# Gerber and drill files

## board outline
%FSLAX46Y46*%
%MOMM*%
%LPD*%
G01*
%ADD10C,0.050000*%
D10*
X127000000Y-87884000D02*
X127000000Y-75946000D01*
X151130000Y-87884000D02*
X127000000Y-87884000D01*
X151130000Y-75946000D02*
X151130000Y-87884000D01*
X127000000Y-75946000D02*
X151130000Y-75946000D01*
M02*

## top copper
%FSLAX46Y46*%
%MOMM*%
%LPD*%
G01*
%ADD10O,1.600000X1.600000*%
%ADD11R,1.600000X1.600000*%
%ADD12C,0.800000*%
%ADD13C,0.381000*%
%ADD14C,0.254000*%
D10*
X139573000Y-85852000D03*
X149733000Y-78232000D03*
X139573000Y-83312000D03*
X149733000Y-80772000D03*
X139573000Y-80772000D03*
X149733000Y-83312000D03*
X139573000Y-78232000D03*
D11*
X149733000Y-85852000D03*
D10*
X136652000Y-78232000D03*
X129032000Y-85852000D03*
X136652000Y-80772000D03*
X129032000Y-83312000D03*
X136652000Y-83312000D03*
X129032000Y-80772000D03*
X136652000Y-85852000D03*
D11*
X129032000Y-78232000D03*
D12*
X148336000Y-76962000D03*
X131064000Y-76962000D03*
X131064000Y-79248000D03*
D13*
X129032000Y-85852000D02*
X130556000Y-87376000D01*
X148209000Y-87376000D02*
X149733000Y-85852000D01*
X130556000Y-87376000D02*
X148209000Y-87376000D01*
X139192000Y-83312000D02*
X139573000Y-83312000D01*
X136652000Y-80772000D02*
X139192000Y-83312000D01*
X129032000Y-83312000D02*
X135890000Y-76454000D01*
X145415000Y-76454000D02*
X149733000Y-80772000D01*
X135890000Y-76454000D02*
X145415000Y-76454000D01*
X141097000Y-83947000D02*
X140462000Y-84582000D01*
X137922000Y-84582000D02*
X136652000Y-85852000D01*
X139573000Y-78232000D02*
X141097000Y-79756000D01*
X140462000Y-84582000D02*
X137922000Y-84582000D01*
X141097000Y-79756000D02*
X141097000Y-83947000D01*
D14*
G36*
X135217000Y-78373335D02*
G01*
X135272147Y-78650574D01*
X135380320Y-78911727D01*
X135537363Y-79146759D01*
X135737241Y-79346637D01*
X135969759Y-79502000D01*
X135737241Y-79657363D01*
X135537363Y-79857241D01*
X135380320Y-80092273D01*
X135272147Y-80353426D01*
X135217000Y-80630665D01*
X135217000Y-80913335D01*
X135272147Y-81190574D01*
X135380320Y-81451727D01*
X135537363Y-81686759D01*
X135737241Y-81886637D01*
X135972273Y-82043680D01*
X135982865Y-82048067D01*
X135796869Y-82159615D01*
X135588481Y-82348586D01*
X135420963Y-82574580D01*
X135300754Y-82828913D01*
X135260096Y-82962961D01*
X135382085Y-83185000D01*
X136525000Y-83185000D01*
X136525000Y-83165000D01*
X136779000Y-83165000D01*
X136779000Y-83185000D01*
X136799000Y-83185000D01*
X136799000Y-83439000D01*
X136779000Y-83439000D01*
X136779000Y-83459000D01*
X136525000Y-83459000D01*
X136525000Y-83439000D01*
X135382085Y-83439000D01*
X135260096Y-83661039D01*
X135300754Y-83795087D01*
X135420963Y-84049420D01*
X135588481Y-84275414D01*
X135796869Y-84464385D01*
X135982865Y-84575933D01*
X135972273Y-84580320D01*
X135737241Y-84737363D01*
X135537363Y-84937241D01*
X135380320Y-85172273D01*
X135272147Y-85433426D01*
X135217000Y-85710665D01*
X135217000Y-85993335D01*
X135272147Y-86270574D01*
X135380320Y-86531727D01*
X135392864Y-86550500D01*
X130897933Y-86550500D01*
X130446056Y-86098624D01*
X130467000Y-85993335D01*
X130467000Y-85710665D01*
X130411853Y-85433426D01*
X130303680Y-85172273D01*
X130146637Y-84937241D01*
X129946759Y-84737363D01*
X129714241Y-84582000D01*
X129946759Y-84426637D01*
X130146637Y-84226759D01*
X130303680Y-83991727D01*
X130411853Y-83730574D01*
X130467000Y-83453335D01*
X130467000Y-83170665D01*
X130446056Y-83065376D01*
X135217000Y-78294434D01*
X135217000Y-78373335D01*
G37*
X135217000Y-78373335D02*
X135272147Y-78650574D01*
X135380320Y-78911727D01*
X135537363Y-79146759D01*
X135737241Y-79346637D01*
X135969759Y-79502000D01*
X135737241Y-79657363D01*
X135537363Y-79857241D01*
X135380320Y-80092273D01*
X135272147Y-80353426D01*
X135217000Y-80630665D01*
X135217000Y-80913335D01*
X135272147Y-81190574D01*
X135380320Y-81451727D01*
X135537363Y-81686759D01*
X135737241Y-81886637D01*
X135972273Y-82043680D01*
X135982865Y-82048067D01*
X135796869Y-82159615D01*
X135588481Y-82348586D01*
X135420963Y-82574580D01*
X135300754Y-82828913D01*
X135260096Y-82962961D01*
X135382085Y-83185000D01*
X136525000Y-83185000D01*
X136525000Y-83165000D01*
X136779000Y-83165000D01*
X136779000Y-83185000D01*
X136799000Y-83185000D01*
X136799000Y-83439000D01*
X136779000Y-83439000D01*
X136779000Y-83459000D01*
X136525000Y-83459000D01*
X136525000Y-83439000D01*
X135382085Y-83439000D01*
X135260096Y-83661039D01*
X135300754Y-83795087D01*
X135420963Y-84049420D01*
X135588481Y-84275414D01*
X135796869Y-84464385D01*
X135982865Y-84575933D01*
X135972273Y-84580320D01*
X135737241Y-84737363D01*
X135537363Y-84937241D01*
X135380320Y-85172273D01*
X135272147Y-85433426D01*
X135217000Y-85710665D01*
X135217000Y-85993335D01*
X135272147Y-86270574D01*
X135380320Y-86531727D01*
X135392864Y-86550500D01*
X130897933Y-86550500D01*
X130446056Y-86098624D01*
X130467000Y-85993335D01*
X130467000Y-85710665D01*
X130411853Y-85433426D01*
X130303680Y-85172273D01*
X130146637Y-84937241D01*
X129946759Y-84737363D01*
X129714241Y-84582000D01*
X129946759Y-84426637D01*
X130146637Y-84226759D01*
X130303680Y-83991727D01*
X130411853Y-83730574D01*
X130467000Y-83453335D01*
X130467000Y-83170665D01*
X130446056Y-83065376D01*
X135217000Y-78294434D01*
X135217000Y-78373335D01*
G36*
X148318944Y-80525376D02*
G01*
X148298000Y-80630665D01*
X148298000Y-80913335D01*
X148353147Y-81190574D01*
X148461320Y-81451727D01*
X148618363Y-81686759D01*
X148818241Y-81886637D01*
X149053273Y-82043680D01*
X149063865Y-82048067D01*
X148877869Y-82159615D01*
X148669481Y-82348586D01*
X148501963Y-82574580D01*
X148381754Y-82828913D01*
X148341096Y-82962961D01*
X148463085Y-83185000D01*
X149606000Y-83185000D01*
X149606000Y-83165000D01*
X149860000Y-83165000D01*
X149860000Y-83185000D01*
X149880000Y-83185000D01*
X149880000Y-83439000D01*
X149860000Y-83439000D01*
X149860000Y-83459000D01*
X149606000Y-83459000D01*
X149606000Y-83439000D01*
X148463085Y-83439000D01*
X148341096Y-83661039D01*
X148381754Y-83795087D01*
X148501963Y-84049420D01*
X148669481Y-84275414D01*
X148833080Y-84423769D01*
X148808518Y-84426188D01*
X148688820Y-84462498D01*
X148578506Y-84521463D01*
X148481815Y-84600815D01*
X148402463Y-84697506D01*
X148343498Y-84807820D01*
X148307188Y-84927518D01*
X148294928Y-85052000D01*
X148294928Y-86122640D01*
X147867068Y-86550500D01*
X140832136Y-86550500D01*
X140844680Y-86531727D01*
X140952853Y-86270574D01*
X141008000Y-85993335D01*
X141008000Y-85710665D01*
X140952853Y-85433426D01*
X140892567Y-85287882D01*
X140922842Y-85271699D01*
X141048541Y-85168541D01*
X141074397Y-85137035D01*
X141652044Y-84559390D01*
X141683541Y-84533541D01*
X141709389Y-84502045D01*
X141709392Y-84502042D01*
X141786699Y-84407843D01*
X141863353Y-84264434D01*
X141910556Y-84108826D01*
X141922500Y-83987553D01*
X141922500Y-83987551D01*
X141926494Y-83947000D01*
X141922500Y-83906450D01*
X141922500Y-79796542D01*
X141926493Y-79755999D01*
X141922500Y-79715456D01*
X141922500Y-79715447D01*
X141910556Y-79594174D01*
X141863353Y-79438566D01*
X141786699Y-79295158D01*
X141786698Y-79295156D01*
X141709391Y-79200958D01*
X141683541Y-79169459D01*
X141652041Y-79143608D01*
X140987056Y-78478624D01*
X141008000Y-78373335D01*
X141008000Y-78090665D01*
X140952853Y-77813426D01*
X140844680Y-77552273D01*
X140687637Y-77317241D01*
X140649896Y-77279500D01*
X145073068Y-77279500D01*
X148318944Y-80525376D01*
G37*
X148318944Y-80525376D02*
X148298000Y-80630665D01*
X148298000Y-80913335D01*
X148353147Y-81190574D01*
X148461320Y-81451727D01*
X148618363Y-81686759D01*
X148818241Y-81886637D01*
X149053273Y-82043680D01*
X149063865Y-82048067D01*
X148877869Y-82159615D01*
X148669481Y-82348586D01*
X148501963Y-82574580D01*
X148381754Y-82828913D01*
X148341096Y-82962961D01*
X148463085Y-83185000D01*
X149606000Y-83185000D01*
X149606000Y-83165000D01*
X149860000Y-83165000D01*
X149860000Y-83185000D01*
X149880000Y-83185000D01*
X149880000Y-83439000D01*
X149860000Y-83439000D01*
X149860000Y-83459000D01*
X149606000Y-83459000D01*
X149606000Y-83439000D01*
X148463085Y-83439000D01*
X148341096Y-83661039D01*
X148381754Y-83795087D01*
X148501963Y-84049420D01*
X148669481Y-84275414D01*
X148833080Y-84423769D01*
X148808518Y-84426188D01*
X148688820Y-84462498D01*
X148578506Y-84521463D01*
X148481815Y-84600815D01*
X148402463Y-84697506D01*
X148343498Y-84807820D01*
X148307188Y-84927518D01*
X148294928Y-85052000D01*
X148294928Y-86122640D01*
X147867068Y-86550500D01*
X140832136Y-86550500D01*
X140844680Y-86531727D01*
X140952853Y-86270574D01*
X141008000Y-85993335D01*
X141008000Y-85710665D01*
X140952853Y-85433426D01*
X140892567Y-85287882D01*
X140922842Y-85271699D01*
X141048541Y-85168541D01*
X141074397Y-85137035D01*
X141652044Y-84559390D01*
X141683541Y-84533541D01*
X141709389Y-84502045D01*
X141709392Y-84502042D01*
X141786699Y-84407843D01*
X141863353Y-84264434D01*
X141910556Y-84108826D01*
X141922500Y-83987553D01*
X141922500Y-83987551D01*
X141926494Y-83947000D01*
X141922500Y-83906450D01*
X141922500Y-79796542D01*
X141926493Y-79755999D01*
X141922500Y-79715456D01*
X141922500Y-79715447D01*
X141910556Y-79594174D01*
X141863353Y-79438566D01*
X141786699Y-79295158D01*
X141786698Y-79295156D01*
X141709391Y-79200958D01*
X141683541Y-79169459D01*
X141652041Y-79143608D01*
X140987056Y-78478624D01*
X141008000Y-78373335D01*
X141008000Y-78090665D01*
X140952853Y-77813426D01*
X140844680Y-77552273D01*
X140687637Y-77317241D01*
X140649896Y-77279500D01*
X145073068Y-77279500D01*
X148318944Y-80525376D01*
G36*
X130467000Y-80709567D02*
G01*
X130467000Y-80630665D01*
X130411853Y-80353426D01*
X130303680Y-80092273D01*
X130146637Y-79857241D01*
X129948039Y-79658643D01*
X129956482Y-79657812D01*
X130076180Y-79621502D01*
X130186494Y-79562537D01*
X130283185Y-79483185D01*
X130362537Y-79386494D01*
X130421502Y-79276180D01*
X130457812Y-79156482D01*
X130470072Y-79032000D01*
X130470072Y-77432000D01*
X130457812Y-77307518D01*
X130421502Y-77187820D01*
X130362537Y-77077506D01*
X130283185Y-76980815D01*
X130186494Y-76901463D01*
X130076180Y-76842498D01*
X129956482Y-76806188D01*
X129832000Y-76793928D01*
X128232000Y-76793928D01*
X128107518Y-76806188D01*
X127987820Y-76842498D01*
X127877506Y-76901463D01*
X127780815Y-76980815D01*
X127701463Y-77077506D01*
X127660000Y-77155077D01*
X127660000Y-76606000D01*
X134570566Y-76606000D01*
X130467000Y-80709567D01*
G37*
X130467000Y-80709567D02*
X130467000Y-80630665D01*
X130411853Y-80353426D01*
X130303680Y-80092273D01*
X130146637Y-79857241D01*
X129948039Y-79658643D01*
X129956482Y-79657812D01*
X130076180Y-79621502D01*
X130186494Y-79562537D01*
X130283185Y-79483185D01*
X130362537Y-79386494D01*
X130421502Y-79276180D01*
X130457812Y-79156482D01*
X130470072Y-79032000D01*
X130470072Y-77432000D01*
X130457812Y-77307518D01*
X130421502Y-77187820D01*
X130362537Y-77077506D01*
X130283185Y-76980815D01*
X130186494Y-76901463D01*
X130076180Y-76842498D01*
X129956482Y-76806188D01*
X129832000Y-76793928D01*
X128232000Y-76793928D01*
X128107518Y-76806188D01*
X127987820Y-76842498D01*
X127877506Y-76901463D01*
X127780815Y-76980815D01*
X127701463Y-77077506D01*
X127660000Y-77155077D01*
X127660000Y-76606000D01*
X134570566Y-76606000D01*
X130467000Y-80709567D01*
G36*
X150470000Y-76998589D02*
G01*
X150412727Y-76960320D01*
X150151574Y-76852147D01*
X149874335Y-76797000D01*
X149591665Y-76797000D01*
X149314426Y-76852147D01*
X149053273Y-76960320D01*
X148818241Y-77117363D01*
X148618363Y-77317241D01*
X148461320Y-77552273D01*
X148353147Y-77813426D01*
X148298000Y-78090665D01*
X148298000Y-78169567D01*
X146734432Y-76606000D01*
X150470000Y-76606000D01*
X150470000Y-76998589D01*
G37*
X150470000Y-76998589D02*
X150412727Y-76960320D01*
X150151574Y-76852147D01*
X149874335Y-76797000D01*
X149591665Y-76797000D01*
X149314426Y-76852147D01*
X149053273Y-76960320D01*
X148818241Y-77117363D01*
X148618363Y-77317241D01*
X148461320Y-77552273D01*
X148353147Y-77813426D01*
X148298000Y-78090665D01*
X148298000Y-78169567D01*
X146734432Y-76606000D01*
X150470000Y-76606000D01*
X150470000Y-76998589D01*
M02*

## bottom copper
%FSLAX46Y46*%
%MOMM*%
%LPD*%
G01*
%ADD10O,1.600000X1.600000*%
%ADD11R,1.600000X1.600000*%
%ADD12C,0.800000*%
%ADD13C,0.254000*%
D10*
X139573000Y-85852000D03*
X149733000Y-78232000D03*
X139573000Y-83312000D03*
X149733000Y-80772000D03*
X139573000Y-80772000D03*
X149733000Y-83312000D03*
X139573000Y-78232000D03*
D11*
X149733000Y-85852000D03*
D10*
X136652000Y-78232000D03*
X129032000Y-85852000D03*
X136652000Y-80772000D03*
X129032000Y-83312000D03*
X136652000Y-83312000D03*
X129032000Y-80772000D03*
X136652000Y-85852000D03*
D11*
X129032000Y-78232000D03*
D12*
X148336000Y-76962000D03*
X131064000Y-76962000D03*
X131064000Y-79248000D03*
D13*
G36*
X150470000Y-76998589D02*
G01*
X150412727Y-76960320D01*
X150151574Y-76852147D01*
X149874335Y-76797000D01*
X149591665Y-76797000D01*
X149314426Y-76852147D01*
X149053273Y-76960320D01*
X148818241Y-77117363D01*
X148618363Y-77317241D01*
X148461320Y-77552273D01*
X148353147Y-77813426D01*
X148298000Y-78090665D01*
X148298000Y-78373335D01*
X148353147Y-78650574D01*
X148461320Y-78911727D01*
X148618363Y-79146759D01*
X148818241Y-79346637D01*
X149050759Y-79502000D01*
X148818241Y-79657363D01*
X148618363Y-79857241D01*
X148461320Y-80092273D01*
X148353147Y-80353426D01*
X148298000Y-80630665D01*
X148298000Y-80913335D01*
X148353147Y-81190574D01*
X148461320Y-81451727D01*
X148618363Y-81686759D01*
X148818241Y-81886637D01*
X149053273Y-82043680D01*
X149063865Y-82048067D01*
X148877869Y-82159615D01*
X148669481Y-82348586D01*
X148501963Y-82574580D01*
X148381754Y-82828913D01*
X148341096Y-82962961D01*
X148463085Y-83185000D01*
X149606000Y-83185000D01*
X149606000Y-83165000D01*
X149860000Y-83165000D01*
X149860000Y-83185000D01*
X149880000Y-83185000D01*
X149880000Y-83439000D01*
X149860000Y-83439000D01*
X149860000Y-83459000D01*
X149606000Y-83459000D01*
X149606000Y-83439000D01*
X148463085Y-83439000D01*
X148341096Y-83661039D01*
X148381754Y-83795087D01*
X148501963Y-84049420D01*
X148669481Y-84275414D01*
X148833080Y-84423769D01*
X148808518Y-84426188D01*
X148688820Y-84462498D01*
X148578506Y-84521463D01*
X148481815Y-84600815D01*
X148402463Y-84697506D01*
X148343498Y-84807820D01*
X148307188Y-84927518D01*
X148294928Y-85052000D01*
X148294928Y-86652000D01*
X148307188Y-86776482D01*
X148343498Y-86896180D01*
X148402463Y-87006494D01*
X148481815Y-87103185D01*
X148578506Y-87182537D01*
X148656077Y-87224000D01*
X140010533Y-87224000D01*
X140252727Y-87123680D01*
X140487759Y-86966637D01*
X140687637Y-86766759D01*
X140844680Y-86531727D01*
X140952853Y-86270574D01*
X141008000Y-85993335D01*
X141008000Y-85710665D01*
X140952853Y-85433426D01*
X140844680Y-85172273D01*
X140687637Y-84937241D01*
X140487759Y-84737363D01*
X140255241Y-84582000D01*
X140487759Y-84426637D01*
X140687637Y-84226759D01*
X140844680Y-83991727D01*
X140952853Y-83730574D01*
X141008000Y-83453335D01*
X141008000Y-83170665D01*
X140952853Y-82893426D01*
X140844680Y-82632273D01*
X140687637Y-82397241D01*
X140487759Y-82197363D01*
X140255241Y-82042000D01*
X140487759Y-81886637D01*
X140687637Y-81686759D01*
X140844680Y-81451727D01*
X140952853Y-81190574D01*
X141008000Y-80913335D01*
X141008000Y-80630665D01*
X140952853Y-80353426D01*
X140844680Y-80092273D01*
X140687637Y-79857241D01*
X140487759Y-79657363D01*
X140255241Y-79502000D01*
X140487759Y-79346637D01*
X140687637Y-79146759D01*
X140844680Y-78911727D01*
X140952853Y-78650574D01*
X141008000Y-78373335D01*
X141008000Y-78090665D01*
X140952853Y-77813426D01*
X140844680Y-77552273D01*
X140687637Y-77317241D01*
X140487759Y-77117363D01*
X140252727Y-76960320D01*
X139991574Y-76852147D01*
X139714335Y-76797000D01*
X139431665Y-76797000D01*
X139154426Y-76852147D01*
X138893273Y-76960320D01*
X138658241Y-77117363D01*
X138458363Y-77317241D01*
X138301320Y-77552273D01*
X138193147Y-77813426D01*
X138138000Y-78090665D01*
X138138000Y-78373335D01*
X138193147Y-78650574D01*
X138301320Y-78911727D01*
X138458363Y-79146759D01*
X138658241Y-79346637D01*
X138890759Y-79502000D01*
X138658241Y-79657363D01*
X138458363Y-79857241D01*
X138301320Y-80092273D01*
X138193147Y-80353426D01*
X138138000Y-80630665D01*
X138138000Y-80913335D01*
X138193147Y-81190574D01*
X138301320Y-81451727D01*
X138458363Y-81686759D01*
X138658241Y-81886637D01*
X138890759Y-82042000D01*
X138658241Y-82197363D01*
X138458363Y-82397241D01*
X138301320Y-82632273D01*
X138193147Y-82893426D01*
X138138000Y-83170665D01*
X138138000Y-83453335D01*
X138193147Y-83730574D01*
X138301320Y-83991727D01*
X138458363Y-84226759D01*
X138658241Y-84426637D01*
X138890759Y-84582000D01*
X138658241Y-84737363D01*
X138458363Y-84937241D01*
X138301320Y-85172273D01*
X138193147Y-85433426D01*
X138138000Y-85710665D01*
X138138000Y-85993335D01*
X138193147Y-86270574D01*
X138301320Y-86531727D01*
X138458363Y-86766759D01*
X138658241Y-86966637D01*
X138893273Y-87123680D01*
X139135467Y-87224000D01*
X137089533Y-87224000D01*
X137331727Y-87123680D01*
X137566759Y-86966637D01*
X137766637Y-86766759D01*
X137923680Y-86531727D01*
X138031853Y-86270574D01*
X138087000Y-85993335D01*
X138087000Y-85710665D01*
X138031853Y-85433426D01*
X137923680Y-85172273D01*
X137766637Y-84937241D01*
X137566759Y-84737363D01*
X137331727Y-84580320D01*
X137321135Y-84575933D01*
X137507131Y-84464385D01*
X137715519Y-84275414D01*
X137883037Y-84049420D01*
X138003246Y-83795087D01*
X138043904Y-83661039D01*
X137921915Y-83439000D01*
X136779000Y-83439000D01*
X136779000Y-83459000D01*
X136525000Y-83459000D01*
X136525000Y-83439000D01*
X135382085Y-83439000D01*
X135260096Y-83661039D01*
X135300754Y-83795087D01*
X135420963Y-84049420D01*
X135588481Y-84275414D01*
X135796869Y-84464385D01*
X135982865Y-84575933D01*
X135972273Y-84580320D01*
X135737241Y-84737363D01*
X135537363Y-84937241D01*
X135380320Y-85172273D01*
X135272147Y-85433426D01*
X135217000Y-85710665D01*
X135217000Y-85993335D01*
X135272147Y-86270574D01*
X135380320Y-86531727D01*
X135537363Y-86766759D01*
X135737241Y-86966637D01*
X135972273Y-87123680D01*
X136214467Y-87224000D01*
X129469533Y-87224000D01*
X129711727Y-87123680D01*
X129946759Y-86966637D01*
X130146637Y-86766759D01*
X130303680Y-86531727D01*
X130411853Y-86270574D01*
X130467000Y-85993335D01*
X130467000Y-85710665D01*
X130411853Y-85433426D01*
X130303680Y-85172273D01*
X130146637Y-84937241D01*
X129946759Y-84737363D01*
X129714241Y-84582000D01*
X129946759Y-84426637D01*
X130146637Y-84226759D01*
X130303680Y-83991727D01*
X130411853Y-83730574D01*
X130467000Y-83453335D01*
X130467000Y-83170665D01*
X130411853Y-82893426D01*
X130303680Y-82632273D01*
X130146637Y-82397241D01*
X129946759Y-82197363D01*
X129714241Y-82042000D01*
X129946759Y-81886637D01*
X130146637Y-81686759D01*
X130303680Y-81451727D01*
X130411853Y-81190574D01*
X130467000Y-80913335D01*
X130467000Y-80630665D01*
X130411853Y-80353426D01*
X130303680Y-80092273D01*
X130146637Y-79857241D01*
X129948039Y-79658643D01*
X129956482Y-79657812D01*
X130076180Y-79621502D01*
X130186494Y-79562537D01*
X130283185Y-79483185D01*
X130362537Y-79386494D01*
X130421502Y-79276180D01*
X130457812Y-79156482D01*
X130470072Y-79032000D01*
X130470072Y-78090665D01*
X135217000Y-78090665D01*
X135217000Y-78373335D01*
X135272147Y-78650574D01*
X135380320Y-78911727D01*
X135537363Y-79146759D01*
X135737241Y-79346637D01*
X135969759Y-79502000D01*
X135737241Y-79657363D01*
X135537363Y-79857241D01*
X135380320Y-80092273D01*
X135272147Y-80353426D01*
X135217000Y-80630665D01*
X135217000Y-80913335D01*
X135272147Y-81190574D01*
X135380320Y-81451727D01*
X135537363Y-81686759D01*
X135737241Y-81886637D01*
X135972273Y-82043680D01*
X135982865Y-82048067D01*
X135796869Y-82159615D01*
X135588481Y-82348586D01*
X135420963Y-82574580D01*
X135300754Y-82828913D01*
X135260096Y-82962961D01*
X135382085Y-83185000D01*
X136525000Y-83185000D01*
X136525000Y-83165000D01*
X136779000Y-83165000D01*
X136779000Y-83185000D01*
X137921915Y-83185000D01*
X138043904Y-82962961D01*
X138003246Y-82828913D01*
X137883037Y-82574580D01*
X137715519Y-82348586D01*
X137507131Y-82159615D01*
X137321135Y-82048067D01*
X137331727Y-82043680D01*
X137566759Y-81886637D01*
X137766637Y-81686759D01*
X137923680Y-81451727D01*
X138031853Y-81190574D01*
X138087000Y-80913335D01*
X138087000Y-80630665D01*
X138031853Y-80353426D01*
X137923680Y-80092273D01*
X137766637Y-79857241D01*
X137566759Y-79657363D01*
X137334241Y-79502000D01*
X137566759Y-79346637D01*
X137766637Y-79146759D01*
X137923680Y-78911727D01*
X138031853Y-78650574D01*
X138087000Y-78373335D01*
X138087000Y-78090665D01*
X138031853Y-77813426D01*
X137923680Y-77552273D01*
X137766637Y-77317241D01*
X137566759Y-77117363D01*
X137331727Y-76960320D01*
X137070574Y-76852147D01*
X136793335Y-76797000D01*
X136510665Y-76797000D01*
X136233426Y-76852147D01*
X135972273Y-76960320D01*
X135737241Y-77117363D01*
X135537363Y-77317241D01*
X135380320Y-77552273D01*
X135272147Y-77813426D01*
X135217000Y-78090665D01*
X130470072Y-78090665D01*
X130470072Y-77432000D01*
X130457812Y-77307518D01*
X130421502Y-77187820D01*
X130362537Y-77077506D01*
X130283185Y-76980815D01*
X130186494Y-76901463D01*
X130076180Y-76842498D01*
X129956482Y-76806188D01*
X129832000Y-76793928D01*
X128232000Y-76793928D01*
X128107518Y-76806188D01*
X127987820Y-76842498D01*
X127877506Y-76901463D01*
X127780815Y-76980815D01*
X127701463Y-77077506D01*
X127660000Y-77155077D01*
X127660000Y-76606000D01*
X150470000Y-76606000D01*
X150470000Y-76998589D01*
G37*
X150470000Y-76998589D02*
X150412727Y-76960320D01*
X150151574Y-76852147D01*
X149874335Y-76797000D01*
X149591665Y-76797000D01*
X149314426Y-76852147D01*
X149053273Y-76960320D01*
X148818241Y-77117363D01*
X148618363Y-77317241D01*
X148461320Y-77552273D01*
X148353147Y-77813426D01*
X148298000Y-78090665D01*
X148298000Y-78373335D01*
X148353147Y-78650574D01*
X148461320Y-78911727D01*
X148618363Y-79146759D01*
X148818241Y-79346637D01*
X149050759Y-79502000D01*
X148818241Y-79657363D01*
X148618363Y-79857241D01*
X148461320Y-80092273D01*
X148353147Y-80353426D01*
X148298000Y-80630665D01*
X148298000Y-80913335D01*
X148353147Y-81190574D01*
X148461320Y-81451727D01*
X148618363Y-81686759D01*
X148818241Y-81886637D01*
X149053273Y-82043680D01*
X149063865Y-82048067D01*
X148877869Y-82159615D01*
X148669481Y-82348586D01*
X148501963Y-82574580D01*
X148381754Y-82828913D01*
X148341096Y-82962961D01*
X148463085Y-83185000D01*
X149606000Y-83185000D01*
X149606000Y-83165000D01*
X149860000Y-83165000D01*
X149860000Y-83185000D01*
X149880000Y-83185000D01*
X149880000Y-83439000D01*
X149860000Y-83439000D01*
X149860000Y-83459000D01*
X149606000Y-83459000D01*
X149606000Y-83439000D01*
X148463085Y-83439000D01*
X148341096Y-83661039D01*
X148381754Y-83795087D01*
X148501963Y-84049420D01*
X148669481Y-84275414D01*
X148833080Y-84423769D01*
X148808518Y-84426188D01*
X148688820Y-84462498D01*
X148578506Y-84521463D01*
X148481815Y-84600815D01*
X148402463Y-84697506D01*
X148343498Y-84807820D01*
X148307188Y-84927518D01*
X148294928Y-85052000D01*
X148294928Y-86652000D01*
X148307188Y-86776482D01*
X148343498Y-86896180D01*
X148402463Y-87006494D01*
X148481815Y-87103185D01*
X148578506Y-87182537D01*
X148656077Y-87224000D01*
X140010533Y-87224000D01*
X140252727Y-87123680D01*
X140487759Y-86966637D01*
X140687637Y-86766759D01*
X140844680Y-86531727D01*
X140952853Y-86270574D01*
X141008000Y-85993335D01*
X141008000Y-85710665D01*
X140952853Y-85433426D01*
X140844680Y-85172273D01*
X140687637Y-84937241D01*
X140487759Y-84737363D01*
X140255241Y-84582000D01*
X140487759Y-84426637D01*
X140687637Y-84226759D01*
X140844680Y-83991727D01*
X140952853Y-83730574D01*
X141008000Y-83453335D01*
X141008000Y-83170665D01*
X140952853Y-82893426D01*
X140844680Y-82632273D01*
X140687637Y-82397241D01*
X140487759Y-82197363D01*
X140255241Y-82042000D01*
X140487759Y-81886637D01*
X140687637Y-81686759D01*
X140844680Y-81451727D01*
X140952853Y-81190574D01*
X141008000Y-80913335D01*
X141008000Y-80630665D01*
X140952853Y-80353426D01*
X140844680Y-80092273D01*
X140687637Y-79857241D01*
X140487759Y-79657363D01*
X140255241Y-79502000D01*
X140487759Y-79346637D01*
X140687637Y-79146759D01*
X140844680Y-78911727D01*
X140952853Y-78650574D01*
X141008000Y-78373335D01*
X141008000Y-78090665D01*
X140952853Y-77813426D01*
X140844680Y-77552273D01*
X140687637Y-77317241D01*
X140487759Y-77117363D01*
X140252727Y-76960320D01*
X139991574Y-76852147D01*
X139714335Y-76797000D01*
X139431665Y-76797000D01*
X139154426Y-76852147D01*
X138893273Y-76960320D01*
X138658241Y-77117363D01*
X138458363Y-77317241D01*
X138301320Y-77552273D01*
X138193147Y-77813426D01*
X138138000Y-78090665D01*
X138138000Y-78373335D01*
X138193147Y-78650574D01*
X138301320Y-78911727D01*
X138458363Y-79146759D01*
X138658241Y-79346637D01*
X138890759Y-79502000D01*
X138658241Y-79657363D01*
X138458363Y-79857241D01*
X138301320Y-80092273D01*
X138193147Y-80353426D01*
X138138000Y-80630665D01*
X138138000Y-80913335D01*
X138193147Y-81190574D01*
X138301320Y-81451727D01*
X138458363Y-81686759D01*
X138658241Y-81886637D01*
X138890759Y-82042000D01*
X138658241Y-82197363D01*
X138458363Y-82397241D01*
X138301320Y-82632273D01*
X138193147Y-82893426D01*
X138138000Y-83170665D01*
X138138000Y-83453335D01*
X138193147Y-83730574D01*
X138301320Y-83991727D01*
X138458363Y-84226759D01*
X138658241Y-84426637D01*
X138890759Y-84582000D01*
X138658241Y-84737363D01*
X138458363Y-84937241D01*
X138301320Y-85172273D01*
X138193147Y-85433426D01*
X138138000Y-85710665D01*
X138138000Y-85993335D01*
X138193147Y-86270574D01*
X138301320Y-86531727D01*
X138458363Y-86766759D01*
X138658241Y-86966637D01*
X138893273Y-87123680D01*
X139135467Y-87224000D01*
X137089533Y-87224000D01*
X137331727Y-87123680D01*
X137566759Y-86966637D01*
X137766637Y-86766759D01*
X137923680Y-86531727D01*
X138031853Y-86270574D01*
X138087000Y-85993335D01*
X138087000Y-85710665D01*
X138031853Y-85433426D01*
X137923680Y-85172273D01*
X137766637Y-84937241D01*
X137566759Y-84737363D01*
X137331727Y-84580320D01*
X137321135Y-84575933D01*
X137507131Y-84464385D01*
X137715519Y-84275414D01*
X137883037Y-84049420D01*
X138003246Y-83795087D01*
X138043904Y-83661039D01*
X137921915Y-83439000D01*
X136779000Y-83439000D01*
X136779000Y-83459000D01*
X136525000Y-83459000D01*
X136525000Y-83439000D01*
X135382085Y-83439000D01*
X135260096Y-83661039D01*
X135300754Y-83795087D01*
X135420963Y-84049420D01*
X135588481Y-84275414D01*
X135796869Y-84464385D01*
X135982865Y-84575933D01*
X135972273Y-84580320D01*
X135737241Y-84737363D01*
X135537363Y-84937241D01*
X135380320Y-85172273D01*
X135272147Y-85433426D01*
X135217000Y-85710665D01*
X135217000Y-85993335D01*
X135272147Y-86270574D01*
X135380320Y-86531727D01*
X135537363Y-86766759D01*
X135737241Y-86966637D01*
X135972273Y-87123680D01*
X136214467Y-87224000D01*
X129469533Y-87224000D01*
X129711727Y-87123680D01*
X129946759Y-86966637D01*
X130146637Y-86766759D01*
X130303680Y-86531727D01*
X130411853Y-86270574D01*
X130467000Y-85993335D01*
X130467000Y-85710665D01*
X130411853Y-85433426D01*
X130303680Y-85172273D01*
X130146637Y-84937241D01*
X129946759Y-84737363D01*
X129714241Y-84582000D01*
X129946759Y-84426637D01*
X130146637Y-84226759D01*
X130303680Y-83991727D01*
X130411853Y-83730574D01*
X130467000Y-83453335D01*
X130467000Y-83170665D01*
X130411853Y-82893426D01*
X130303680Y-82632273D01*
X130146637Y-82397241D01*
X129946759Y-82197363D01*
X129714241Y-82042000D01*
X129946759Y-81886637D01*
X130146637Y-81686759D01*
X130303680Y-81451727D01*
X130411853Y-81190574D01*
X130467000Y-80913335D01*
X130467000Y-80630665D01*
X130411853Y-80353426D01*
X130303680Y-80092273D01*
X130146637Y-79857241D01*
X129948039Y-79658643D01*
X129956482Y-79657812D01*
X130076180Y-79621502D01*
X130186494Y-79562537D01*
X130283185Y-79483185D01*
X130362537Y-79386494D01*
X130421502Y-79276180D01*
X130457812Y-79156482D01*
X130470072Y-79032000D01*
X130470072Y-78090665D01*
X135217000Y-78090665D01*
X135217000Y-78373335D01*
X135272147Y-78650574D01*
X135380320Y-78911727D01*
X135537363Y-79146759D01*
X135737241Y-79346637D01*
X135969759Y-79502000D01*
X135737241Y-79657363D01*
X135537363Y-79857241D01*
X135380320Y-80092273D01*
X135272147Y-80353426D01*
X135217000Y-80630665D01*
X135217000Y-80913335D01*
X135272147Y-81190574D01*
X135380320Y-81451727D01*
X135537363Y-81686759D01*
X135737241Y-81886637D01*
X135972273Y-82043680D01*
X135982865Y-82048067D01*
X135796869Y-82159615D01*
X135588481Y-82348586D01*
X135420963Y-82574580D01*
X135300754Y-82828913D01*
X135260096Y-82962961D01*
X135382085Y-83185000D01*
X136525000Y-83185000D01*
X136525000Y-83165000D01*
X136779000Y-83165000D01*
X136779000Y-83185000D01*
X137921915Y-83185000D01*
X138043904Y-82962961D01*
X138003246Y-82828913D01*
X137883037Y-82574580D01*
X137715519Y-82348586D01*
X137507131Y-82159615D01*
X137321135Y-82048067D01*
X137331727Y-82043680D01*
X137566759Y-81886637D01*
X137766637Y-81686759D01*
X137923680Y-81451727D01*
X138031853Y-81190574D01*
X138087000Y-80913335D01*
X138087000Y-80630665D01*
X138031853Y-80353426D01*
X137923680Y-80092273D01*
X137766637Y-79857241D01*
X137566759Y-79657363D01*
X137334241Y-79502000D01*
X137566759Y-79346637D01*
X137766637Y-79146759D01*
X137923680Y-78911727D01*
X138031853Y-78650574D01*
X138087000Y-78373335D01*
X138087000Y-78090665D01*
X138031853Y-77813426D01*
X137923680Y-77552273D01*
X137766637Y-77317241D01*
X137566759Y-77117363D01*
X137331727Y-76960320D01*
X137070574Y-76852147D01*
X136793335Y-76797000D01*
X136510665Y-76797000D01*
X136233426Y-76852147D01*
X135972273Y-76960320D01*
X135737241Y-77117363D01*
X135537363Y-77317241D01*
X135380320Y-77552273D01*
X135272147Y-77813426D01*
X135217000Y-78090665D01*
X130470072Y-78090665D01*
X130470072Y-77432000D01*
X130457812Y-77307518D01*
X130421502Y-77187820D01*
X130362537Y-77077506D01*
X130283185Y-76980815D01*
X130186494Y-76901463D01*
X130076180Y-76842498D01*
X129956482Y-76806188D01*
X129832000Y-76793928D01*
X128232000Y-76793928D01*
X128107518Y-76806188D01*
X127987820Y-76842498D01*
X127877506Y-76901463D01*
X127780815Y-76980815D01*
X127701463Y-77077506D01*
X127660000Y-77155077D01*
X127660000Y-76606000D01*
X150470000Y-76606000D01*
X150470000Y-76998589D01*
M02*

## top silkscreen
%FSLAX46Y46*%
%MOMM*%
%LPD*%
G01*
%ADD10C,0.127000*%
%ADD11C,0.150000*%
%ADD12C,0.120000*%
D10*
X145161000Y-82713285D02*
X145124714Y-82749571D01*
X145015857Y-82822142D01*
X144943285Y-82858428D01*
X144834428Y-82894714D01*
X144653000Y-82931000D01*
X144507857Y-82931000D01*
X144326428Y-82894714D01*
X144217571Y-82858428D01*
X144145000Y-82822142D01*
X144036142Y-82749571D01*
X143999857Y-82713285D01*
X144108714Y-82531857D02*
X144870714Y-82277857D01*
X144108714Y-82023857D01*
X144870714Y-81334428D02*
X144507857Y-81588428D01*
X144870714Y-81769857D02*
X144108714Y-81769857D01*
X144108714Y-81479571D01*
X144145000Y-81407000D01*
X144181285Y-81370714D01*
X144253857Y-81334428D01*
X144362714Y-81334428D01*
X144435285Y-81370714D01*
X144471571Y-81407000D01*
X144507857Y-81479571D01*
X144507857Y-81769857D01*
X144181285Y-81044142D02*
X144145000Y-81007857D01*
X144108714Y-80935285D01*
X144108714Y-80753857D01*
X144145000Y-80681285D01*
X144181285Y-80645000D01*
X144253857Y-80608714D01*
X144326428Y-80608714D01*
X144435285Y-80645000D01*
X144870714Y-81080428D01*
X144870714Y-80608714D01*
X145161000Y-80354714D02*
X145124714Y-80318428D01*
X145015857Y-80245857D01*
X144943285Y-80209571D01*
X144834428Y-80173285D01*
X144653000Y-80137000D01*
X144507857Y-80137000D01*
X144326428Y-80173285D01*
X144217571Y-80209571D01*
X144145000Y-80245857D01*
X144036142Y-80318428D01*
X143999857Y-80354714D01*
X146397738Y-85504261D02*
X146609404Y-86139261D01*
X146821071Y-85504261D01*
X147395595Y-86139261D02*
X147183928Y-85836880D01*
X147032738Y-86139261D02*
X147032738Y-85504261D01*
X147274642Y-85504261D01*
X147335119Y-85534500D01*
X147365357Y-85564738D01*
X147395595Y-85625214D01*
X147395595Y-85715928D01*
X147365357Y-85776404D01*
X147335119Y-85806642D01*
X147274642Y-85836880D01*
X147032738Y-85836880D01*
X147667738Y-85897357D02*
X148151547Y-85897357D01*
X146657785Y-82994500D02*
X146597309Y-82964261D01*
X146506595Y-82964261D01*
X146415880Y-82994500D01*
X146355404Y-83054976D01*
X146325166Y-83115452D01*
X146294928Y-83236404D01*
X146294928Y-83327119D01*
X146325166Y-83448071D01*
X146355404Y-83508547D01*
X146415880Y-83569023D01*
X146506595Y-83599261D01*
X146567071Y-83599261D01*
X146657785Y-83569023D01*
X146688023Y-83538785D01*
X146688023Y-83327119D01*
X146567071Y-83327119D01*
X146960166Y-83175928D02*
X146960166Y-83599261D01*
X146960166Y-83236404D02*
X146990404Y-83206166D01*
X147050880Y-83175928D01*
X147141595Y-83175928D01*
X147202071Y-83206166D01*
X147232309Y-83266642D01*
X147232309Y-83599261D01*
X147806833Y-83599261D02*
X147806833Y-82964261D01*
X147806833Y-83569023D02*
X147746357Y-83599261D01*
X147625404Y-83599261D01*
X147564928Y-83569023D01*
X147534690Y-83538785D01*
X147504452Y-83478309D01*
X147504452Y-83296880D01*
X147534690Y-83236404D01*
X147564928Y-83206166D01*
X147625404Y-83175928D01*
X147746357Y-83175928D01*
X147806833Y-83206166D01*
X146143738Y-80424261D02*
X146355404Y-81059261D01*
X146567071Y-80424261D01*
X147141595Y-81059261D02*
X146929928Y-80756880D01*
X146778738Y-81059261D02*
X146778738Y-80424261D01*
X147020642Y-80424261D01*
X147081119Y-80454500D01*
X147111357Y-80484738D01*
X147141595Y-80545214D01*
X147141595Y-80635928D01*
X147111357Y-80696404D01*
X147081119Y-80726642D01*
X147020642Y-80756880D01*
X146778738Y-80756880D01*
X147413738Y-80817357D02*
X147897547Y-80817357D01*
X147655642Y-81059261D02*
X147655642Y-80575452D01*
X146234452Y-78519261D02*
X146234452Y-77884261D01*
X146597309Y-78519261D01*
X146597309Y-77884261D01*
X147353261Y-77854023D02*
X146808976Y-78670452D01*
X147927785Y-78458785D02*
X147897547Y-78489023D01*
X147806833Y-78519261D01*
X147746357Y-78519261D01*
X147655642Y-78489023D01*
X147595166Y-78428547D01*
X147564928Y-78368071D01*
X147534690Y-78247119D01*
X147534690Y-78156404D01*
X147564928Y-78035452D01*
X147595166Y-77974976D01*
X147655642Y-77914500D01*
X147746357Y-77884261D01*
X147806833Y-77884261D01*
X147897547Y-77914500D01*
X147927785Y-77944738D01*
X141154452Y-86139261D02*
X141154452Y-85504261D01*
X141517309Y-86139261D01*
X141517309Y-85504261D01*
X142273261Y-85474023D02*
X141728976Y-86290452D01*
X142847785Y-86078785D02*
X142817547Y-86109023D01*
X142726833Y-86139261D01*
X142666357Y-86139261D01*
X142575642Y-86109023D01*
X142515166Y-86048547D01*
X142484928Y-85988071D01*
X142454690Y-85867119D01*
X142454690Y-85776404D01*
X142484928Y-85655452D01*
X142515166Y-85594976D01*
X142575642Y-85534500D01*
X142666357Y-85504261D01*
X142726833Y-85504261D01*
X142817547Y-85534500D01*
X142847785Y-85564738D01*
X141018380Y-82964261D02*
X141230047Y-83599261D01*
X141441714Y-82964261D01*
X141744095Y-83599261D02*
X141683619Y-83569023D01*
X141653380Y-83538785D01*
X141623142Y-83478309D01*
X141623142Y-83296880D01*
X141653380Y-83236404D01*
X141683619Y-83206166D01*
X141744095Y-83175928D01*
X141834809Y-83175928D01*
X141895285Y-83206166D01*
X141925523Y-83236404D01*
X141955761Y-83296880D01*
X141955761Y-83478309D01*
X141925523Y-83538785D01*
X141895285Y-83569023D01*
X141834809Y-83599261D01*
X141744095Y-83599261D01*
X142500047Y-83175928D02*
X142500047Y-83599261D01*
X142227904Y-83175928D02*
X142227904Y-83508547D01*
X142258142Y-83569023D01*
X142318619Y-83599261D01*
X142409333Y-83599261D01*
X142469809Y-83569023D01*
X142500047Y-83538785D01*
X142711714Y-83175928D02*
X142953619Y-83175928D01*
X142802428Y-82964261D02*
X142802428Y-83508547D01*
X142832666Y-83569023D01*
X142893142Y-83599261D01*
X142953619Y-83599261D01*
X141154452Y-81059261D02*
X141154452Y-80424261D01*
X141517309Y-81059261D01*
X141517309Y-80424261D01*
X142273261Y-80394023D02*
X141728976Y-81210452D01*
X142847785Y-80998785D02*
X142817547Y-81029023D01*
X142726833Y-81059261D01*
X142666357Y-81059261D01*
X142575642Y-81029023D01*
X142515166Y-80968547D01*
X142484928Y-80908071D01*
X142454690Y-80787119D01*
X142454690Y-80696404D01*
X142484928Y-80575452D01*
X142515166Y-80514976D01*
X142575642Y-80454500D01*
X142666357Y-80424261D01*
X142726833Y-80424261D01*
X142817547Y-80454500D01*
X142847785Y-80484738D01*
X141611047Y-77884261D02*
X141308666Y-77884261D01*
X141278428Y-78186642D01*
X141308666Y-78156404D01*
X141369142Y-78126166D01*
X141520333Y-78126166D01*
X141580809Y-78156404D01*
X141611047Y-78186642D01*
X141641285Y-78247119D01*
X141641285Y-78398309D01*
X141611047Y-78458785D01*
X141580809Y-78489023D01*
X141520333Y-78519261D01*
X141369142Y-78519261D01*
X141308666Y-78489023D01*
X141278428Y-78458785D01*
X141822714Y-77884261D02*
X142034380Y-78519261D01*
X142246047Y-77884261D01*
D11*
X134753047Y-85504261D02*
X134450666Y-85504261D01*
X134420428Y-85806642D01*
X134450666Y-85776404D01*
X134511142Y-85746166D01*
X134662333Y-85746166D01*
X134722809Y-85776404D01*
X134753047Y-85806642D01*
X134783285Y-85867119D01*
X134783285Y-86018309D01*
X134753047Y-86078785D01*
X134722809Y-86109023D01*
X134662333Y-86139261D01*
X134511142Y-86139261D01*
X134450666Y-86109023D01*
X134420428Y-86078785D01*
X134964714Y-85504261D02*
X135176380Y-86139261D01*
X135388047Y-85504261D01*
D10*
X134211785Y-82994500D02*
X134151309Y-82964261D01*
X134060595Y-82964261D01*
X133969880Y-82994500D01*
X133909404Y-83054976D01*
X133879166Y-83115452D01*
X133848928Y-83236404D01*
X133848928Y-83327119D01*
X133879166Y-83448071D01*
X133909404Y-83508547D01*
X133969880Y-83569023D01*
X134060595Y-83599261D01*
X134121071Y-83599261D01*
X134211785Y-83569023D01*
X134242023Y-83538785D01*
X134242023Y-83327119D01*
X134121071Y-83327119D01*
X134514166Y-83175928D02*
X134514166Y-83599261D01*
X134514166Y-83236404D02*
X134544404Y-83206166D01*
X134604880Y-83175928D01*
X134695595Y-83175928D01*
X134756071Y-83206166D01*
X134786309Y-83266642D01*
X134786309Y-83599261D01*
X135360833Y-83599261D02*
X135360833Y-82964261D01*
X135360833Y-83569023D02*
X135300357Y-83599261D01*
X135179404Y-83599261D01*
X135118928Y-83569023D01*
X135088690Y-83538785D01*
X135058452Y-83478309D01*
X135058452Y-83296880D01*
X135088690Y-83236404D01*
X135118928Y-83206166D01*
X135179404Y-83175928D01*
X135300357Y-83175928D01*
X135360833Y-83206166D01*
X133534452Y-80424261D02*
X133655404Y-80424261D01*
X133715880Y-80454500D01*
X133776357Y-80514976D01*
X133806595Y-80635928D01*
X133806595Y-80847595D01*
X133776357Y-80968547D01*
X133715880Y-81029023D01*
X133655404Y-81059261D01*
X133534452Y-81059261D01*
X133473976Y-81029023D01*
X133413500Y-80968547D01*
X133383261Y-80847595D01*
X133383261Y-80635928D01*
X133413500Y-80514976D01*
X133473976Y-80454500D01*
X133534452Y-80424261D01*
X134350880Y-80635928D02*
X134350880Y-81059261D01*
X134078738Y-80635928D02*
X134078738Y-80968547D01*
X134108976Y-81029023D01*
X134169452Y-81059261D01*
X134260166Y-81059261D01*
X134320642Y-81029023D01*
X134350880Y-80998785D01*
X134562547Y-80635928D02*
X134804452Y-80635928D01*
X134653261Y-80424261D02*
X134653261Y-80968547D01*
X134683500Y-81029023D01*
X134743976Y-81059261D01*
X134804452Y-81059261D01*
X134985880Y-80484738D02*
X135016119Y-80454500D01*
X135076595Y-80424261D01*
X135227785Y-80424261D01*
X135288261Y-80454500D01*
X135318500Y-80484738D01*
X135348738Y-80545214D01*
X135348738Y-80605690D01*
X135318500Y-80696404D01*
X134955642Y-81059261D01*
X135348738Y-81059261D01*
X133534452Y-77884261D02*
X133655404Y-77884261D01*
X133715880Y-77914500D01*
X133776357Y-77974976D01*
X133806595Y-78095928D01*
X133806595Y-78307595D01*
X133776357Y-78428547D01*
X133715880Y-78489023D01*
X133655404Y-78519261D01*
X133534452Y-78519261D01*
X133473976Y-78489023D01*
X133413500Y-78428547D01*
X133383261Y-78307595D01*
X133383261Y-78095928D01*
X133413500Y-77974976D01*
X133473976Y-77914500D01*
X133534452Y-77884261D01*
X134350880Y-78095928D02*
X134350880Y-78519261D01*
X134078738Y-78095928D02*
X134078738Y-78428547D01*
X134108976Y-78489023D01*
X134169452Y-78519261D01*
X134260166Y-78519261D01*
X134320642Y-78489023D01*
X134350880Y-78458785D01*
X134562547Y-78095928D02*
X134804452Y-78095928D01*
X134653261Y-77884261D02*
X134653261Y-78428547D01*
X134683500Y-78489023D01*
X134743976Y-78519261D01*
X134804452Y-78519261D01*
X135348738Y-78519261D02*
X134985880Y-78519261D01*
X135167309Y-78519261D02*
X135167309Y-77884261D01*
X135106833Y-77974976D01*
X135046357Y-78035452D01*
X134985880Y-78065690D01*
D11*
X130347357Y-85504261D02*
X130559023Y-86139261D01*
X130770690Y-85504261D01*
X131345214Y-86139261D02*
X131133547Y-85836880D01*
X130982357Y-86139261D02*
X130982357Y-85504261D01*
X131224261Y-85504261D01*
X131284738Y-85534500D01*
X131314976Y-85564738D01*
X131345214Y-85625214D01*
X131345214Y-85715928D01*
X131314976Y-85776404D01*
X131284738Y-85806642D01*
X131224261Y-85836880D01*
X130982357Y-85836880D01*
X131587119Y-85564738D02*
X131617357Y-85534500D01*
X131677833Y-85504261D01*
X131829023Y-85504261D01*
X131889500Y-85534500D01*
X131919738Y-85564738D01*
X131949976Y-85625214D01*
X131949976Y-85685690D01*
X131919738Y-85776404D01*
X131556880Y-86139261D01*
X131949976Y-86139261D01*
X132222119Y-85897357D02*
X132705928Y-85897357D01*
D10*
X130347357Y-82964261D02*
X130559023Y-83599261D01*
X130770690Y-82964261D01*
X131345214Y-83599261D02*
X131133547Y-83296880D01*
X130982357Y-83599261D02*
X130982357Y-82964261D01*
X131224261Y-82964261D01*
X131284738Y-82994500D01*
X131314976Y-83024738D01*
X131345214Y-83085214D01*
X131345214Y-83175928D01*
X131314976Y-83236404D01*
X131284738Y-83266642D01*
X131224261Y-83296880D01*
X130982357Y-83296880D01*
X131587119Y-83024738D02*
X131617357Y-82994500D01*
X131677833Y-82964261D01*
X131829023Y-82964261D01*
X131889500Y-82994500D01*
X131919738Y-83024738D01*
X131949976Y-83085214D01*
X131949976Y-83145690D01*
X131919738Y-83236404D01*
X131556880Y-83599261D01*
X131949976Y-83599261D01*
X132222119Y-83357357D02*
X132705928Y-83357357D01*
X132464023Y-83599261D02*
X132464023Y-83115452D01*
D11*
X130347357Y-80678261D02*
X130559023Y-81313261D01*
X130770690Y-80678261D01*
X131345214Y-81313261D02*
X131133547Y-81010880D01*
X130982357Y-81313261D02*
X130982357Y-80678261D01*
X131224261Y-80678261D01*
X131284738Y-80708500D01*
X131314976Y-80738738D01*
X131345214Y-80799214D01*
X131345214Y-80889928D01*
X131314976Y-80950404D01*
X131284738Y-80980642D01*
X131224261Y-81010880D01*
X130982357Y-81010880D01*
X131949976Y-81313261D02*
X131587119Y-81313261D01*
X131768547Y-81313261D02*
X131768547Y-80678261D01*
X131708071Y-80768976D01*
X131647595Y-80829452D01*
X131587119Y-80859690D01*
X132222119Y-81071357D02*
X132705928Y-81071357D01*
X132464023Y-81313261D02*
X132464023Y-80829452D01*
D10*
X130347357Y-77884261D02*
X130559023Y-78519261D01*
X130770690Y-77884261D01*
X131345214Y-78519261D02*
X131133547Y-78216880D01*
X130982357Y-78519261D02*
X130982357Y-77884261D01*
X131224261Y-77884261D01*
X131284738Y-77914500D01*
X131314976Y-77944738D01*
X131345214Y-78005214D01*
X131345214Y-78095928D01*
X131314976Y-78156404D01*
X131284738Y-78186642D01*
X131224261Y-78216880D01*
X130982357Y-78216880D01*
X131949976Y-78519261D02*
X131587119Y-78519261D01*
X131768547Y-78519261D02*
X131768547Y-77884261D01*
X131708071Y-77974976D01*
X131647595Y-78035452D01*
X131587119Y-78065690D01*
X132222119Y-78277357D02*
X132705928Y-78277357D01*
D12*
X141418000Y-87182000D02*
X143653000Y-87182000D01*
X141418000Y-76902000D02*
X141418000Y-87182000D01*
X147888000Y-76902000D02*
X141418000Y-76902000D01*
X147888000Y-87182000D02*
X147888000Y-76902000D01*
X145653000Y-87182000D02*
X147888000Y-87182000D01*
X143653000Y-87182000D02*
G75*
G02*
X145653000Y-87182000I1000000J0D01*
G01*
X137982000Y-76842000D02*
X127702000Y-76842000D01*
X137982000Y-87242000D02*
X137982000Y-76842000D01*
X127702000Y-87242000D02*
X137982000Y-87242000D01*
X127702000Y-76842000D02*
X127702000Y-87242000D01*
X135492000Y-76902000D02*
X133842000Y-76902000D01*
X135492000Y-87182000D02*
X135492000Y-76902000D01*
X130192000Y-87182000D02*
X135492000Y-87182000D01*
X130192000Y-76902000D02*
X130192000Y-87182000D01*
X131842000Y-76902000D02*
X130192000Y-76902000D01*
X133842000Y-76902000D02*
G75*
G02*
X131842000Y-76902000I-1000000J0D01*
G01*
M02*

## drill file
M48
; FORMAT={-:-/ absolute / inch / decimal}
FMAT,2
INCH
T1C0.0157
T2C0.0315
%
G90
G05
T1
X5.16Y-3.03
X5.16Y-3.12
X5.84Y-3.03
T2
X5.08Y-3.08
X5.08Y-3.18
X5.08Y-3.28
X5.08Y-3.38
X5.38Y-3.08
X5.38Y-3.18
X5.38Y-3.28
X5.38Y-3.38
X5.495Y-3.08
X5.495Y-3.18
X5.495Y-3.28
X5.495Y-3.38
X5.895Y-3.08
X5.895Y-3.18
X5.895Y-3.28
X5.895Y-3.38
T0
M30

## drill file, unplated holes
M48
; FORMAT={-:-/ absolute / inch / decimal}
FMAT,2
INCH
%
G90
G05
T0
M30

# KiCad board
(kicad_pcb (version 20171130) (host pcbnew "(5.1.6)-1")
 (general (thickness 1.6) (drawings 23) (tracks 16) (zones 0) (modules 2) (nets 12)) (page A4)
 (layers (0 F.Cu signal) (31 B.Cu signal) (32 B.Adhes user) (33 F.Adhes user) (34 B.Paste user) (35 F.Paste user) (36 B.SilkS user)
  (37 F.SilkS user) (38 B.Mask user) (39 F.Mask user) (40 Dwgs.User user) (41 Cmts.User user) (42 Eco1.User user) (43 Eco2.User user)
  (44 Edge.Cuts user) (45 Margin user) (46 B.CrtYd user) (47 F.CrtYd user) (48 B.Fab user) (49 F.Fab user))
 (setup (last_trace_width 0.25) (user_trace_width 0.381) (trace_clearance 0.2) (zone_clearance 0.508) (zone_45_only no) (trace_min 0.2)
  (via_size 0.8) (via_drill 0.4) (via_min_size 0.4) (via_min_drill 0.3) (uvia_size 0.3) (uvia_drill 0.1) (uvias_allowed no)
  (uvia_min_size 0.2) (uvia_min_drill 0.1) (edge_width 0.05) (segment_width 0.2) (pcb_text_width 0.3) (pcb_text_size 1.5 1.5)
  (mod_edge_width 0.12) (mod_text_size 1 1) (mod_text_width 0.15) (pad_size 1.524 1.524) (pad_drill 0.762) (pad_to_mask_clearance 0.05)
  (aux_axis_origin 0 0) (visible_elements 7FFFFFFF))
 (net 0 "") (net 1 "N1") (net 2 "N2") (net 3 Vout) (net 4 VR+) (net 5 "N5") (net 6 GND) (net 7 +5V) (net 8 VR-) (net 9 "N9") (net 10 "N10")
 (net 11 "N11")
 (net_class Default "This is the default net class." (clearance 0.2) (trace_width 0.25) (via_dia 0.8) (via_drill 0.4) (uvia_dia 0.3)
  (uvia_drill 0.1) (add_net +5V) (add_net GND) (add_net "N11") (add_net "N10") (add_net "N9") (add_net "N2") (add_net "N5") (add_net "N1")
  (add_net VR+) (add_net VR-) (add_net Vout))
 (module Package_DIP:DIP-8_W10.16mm (layer F.Cu) (at 149.733 85.852 180)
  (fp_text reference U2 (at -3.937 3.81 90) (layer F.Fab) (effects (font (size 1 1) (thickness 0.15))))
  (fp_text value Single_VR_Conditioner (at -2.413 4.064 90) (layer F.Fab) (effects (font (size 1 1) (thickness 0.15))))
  (fp_line (start 8.315 -1.33) (end 6.08 -1.33) (layer F.SilkS) (width 0.12))
  (fp_line (start 8.315 8.95) (end 8.315 -1.33) (layer F.SilkS) (width 0.12))
  (fp_line (start 1.845 8.95) (end 8.315 8.95) (layer F.SilkS) (width 0.12))
  (fp_line (start 1.845 -1.33) (end 1.845 8.95) (layer F.SilkS) (width 0.12))
  (fp_line (start 4.08 -1.33) (end 1.845 -1.33) (layer F.SilkS) (width 0.12))
  (fp_arc (start 5.08 -1.33) (end 4.08 -1.33) (angle -180) (layer F.SilkS) (width 0.12))
  (pad 8 thru_hole oval (at 10.16 0 180) (size 1.6 1.6) (drill 0.8) (layers *.Cu *.Mask) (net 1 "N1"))
  (pad 4 thru_hole oval (at 0 7.62 180) (size 1.6 1.6) (drill 0.8) (layers *.Cu *.Mask) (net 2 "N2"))
  (pad 7 thru_hole oval (at 10.16 2.54 180) (size 1.6 1.6) (drill 0.8) (layers *.Cu *.Mask) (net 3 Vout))
  (pad 3 thru_hole oval (at 0 5.08 180) (size 1.6 1.6) (drill 0.8) (layers *.Cu *.Mask) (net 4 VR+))
  (pad 6 thru_hole oval (at 10.16 5.08 180) (size 1.6 1.6) (drill 0.8) (layers *.Cu *.Mask) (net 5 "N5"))
  (pad 2 thru_hole oval (at 0 2.54 180) (size 1.6 1.6) (drill 0.8) (layers *.Cu *.Mask) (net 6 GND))
  (pad 5 thru_hole oval (at 10.16 7.62 180) (size 1.6 1.6) (drill 0.8) (layers *.Cu *.Mask) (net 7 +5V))
  (pad 1 thru_hole rect (at 0 0 180) (size 1.6 1.6) (drill 0.8) (layers *.Cu *.Mask) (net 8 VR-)))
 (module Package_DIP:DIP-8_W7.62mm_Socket (layer F.Cu) (at 129.032 78.232)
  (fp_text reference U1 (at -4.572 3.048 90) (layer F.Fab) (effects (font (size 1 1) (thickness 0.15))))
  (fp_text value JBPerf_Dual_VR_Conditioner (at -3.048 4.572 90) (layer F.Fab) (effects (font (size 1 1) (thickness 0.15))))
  (fp_line (start 8.95 -1.39) (end -1.33 -1.39) (layer F.SilkS) (width 0.12))
  (fp_line (start 8.95 9.01) (end 8.95 -1.39) (layer F.SilkS) (width 0.12))
  (fp_line (start -1.33 9.01) (end 8.95 9.01) (layer F.SilkS) (width 0.12))
  (fp_line (start -1.33 -1.39) (end -1.33 9.01) (layer F.SilkS) (width 0.12))
  (fp_line (start 6.46 -1.33) (end 4.81 -1.33) (layer F.SilkS) (width 0.12))
  (fp_line (start 6.46 8.95) (end 6.46 -1.33) (layer F.SilkS) (width 0.12))
  (fp_line (start 1.16 8.95) (end 6.46 8.95) (layer F.SilkS) (width 0.12))
  (fp_line (start 1.16 -1.33) (end 1.16 8.95) (layer F.SilkS) (width 0.12))
  (fp_line (start 2.81 -1.33) (end 1.16 -1.33) (layer F.SilkS) (width 0.12))
  (fp_arc (start 3.81 -1.33) (end 2.81 -1.33) (angle -180) (layer F.SilkS) (width 0.12))
  (pad 8 thru_hole oval (at 7.62 0) (size 1.6 1.6) (drill 0.8) (layers *.Cu *.Mask) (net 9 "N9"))
  (pad 4 thru_hole oval (at 0 7.62) (size 1.6 1.6) (drill 0.8) (layers *.Cu *.Mask) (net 8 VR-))
  (pad 7 thru_hole oval (at 7.62 2.54) (size 1.6 1.6) (drill 0.8) (layers *.Cu *.Mask) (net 3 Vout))
  (pad 3 thru_hole oval (at 0 5.08) (size 1.6 1.6) (drill 0.8) (layers *.Cu *.Mask) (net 4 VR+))
  (pad 6 thru_hole oval (at 7.62 5.08) (size 1.6 1.6) (drill 0.8) (layers *.Cu *.Mask) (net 6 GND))
  (pad 2 thru_hole oval (at 0 2.54) (size 1.6 1.6) (drill 0.8) (layers *.Cu *.Mask) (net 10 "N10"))
  (pad 5 thru_hole oval (at 7.62 7.62) (size 1.6 1.6) (drill 0.8) (layers *.Cu *.Mask) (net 7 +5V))
  (pad 1 thru_hole rect (at 0 0) (size 1.6 1.6) (drill 0.8) (layers *.Cu *.Mask) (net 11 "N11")))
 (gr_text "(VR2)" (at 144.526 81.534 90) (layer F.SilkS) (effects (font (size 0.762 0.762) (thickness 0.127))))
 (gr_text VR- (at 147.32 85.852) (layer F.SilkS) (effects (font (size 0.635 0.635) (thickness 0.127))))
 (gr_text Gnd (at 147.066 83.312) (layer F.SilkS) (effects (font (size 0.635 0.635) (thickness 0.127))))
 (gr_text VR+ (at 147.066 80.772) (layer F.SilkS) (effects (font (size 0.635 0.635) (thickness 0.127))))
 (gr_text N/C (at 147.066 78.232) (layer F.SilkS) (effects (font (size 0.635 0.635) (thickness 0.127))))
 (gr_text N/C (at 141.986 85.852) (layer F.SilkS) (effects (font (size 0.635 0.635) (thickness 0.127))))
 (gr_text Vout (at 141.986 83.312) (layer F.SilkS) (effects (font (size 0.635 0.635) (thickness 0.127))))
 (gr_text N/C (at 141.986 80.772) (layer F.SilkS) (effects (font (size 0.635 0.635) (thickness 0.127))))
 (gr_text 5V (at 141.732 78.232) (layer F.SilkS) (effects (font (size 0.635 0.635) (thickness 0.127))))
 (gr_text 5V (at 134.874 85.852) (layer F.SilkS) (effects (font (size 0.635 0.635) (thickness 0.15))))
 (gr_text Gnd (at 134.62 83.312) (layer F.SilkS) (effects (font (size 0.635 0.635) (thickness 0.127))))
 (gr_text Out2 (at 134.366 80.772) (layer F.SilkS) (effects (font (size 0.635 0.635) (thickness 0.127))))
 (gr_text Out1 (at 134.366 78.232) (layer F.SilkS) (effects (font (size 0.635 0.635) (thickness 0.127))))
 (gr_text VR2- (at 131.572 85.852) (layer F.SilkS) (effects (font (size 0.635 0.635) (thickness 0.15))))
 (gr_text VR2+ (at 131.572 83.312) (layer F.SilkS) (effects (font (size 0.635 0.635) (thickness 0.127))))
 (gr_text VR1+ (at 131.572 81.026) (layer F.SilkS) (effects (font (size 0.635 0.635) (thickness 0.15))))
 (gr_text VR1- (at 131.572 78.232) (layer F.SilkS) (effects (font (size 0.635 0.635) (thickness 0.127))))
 (gr_line (start 127 87.884) (end 127 75.946) (layer Edge.Cuts) (width 0.05))
 (gr_line (start 151.13 87.884) (end 127 87.884) (layer Edge.Cuts) (width 0.05))
 (gr_line (start 151.13 75.946) (end 151.13 87.884) (layer Edge.Cuts) (width 0.05))
 (gr_line (start 127 75.946) (end 151.13 75.946) (layer Edge.Cuts) (width 0.05))
 (segment (start 129.032 85.852) (end 130.556 87.376) (width 0.381) (layer F.Cu) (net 8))
 (segment (start 148.209 87.376) (end 149.733 85.852) (width 0.381) (layer F.Cu) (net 8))
 (segment (start 130.556 87.376) (end 148.209 87.376) (width 0.381) (layer F.Cu) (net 8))
 (segment (start 139.192 83.312) (end 139.573 83.312) (width 0.381) (layer F.Cu) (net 3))
 (segment (start 136.652 80.772) (end 139.192 83.312) (width 0.381) (layer F.Cu) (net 3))
 (segment (start 129.032 83.312) (end 135.89 76.454) (width 0.381) (layer F.Cu) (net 4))
 (segment (start 145.415 76.454) (end 149.733 80.772) (width 0.381) (layer F.Cu) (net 4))
 (segment (start 135.89 76.454) (end 145.415 76.454) (width 0.381) (layer F.Cu) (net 4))
 (via (at 148.336 76.962) (size 0.8) (drill 0.4) (layers F.Cu B.Cu) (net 6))
 (via (at 131.064 76.962) (size 0.8) (drill 0.4) (layers F.Cu B.Cu) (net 6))
 (via (at 131.064 79.248) (size 0.8) (drill 0.4) (layers F.Cu B.Cu) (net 6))
 (segment (start 141.097 83.947) (end 140.462 84.582) (width 0.381) (layer F.Cu) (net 7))
 (segment (start 137.922 84.582) (end 136.652 85.852) (width 0.381) (layer F.Cu) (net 7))
 (segment (start 139.573 78.232) (end 141.097 79.756) (width 0.381) (layer F.Cu) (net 7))
 (segment (start 140.462 84.582) (end 137.922 84.582) (width 0.381) (layer F.Cu) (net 7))
 (segment (start 141.097 79.756) (end 141.097 83.947) (width 0.381) (layer F.Cu) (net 7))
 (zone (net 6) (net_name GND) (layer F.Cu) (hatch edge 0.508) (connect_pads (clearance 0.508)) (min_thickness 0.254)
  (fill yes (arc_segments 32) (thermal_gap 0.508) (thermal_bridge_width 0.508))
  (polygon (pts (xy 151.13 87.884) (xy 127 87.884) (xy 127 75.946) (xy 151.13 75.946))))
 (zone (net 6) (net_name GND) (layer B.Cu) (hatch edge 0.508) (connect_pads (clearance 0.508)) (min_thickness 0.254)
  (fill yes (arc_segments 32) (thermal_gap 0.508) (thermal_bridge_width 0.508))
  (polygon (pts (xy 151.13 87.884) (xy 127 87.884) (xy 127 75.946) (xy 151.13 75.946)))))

